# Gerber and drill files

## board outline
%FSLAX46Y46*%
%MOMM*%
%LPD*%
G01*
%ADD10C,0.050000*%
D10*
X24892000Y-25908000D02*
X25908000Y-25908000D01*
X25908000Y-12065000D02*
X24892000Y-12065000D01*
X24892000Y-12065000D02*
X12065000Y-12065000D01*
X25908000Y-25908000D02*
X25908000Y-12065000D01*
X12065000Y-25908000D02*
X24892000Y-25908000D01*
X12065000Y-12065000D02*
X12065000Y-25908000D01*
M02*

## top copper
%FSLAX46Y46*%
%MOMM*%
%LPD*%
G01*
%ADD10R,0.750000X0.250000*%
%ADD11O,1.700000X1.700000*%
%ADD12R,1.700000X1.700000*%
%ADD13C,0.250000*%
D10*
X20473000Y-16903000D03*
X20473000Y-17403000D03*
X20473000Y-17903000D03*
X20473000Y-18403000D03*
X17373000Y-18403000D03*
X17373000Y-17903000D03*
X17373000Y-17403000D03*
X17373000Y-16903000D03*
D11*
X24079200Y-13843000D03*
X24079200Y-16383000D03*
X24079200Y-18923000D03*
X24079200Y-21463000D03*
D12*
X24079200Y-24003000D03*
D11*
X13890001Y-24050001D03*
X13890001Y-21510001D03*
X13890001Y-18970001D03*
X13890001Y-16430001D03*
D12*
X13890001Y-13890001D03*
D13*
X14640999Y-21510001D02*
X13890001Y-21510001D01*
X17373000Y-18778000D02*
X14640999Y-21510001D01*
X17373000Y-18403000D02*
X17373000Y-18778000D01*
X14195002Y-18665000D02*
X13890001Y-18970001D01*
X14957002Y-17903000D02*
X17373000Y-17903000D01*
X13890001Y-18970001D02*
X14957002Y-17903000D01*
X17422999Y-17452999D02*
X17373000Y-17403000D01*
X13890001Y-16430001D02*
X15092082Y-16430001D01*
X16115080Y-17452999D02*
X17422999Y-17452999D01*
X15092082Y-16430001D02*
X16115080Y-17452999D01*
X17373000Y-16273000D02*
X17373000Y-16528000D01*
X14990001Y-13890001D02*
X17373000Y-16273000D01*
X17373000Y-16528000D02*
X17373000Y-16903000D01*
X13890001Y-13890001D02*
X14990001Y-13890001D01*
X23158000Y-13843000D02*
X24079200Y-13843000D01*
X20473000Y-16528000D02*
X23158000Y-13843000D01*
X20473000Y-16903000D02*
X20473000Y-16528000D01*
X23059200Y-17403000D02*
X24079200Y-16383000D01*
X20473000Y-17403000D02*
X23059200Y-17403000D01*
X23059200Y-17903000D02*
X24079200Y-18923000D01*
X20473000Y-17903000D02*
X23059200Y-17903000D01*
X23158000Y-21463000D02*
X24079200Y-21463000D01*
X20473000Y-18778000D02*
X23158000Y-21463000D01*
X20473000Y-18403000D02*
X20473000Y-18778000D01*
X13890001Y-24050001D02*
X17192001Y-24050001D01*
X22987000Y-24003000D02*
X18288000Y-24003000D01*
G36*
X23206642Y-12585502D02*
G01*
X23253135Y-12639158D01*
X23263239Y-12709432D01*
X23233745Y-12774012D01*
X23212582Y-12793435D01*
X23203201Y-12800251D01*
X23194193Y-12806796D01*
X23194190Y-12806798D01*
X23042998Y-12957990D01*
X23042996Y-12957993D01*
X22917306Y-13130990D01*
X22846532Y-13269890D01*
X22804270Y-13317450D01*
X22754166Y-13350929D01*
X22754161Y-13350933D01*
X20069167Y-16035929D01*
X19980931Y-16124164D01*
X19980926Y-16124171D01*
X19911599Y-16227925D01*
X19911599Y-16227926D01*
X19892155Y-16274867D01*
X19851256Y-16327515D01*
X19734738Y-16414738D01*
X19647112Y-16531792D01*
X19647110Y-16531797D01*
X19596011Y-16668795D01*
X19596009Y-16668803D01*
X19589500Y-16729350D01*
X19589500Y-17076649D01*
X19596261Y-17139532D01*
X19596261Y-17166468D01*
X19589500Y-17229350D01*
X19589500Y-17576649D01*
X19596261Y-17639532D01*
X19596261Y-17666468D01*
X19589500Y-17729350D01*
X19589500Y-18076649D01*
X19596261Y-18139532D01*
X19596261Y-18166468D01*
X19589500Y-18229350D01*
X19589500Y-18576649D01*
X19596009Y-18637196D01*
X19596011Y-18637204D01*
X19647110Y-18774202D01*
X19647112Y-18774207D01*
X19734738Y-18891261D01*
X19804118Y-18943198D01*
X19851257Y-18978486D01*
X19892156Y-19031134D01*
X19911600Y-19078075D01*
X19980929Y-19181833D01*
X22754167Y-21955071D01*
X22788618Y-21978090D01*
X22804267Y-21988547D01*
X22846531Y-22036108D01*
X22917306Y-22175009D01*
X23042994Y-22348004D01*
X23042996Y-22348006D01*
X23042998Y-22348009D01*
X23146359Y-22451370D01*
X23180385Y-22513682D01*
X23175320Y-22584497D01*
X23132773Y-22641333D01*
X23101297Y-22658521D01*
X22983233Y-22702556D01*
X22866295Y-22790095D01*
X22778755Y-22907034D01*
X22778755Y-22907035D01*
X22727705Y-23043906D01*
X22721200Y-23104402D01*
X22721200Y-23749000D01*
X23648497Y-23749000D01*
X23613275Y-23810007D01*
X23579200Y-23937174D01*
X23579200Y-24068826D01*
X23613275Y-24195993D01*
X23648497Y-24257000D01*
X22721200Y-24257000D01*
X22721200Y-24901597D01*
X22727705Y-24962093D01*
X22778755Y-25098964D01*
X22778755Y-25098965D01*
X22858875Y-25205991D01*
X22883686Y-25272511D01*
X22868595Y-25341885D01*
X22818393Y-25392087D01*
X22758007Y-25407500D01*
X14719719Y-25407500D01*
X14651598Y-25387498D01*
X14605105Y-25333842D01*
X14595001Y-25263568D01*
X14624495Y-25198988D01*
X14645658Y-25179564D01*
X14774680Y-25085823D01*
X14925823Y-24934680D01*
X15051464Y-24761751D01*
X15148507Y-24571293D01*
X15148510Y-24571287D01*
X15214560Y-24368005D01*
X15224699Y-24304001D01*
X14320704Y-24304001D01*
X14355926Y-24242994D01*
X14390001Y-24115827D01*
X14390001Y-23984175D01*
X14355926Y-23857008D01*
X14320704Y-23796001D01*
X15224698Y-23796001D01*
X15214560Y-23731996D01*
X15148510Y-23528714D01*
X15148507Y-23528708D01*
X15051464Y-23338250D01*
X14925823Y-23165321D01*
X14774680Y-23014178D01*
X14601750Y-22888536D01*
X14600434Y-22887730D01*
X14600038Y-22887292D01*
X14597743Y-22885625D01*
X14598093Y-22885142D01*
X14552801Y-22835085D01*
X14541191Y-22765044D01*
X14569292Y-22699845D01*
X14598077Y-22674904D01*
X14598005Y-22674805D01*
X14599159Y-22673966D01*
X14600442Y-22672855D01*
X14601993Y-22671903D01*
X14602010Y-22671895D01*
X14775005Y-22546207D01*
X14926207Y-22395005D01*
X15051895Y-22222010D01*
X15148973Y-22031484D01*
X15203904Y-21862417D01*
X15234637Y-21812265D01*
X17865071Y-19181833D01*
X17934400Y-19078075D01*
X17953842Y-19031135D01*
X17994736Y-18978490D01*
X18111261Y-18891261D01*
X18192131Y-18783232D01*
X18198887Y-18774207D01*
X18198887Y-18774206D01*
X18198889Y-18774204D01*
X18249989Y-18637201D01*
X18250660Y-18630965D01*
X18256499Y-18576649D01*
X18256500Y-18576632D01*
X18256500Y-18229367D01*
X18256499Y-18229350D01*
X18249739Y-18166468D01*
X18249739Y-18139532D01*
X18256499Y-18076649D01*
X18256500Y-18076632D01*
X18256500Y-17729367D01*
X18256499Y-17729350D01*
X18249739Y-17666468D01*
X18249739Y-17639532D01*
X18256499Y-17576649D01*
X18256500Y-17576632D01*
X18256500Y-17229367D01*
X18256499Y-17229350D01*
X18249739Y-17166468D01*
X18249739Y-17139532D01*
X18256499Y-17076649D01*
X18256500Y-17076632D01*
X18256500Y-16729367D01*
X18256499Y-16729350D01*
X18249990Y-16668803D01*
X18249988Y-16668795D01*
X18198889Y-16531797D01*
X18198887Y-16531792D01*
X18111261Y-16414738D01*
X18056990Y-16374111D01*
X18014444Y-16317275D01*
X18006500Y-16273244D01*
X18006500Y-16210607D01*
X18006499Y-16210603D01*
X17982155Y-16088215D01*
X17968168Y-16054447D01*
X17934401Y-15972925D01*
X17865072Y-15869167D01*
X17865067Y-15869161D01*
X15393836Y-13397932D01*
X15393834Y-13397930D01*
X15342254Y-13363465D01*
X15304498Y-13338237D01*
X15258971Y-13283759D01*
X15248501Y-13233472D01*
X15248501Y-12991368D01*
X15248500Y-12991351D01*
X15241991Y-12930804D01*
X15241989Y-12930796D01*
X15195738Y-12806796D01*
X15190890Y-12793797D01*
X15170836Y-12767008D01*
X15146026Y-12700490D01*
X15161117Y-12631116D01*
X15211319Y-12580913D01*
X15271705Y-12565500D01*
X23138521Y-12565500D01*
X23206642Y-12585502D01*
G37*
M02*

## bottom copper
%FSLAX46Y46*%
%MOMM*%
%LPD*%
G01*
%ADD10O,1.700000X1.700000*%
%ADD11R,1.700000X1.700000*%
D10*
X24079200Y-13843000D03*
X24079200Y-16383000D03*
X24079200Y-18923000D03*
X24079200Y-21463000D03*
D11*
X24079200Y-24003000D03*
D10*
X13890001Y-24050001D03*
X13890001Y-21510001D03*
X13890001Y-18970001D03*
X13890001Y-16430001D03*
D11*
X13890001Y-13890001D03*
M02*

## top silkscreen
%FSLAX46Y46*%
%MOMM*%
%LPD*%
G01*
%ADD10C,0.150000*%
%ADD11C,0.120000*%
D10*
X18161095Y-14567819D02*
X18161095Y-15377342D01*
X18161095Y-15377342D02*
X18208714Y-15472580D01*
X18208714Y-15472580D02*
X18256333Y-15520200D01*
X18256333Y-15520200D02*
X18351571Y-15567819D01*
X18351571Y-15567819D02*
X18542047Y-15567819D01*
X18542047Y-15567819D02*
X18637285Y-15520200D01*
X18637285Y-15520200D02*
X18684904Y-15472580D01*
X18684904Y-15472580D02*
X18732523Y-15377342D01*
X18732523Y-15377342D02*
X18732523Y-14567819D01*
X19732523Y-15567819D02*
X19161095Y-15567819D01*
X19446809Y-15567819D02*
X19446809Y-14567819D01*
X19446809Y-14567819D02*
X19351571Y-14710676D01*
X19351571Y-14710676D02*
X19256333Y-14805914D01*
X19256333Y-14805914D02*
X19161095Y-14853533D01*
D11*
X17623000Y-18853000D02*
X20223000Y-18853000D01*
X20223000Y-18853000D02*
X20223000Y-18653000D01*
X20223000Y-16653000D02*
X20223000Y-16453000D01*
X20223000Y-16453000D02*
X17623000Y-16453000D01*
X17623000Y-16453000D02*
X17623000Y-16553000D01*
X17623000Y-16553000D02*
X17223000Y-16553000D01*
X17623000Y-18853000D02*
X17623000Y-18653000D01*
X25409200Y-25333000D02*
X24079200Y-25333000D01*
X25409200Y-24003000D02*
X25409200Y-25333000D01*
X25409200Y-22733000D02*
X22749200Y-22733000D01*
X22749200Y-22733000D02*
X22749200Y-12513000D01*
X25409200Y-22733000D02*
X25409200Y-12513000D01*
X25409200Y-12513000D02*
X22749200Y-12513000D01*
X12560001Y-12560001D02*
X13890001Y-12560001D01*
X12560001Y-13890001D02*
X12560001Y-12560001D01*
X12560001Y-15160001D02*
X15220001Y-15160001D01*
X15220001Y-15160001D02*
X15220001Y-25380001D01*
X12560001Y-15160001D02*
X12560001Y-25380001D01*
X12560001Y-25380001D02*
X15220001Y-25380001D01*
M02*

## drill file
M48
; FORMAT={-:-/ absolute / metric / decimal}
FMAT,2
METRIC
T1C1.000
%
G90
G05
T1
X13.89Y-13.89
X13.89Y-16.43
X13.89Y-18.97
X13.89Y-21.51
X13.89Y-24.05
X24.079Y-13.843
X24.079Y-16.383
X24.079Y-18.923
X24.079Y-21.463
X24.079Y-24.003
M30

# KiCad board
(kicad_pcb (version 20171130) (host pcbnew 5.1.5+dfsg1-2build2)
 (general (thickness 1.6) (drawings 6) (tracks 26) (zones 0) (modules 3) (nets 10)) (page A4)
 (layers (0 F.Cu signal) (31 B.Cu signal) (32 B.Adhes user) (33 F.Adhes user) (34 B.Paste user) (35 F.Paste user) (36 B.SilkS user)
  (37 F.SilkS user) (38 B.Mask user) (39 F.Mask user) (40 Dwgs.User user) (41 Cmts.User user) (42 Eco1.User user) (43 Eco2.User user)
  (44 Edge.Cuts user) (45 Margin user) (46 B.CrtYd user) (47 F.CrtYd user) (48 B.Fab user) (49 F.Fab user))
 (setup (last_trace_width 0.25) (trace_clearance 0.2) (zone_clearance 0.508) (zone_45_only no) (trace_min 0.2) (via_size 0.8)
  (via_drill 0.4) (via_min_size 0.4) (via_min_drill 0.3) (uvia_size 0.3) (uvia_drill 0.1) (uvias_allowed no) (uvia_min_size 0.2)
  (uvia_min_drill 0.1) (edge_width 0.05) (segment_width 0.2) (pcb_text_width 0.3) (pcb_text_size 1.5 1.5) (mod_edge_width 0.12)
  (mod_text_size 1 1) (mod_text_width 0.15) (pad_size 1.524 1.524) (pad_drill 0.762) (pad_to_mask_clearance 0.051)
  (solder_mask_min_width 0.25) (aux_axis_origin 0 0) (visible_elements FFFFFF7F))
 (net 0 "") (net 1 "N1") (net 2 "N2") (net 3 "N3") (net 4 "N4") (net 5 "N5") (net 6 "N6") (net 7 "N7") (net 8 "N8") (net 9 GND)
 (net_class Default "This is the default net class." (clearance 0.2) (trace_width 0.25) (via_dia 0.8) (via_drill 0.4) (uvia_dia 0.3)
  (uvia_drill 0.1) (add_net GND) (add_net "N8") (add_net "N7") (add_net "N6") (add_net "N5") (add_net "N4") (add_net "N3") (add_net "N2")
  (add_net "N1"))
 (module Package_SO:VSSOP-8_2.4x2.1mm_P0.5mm (layer F.Cu) (at 18.923 17.653)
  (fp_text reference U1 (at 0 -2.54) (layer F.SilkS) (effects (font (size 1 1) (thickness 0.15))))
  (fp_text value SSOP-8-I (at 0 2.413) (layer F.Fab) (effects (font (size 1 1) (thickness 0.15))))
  (fp_line (start -1.3 1.2) (end 1.3 1.2) (layer F.SilkS) (width 0.12))
  (fp_line (start 1.3 1.2) (end 1.3 1) (layer F.SilkS) (width 0.12))
  (fp_line (start 1.3 -1) (end 1.3 -1.2) (layer F.SilkS) (width 0.12))
  (fp_line (start 1.3 -1.2) (end -1.3 -1.2) (layer F.SilkS) (width 0.12))
  (fp_line (start -1.3 -1.2) (end -1.3 -1.1) (layer F.SilkS) (width 0.12))
  (fp_line (start -1.3 -1.1) (end -1.7 -1.1) (layer F.SilkS) (width 0.12))
  (fp_line (start -1.3 1.2) (end -1.3 1) (layer F.SilkS) (width 0.12))
  (pad 8 smd rect (at 1.55 -0.75) (size 0.75 0.25) (layers F.Cu F.Paste F.Mask) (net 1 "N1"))
  (pad 7 smd rect (at 1.55 -0.25) (size 0.75 0.25) (layers F.Cu F.Paste F.Mask) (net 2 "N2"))
  (pad 6 smd rect (at 1.55 0.25) (size 0.75 0.25) (layers F.Cu F.Paste F.Mask) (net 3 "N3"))
  (pad 5 smd rect (at 1.55 0.75) (size 0.75 0.25) (layers F.Cu F.Paste F.Mask) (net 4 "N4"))
  (pad 4 smd rect (at -1.55 0.75) (size 0.75 0.25) (layers F.Cu F.Paste F.Mask) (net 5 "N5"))
  (pad 3 smd rect (at -1.55 0.25) (size 0.75 0.25) (layers F.Cu F.Paste F.Mask) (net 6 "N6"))
  (pad 2 smd rect (at -1.55 -0.25) (size 0.75 0.25) (layers F.Cu F.Paste F.Mask) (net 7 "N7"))
  (pad 1 smd rect (at -1.55 -0.75) (size 0.75 0.25) (layers F.Cu F.Paste F.Mask) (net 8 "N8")))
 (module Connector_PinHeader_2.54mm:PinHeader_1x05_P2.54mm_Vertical (layer F.Cu) (at 24.0792 24.003 180)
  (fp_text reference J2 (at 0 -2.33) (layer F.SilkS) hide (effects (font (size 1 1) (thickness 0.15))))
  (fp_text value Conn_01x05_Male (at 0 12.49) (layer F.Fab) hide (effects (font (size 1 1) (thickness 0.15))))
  (fp_line (start -1.33 -1.33) (end 0 -1.33) (layer F.SilkS) (width 0.12))
  (fp_line (start -1.33 0) (end -1.33 -1.33) (layer F.SilkS) (width 0.12))
  (fp_line (start -1.33 1.27) (end 1.33 1.27) (layer F.SilkS) (width 0.12))
  (fp_line (start 1.33 1.27) (end 1.33 11.49) (layer F.SilkS) (width 0.12))
  (fp_line (start -1.33 1.27) (end -1.33 11.49) (layer F.SilkS) (width 0.12))
  (fp_line (start -1.33 11.49) (end 1.33 11.49) (layer F.SilkS) (width 0.12))
  (pad 5 thru_hole oval (at 0 10.16 180) (size 1.7 1.7) (drill 1) (layers *.Cu *.Mask) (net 1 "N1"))
  (pad 4 thru_hole oval (at 0 7.62 180) (size 1.7 1.7) (drill 1) (layers *.Cu *.Mask) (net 2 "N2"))
  (pad 3 thru_hole oval (at 0 5.08 180) (size 1.7 1.7) (drill 1) (layers *.Cu *.Mask) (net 3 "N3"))
  (pad 2 thru_hole oval (at 0 2.54 180) (size 1.7 1.7) (drill 1) (layers *.Cu *.Mask) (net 4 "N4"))
  (pad 1 thru_hole rect (at 0 0 180) (size 1.7 1.7) (drill 1) (layers *.Cu *.Mask) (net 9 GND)))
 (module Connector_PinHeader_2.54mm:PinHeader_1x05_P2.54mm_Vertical (layer F.Cu) (at 13.890001 13.890001)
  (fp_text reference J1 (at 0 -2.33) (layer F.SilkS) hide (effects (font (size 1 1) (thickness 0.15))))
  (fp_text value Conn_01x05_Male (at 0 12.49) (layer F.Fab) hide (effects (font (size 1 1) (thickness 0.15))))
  (fp_line (start -1.33 -1.33) (end 0 -1.33) (layer F.SilkS) (width 0.12))
  (fp_line (start -1.33 0) (end -1.33 -1.33) (layer F.SilkS) (width 0.12))
  (fp_line (start -1.33 1.27) (end 1.33 1.27) (layer F.SilkS) (width 0.12))
  (fp_line (start 1.33 1.27) (end 1.33 11.49) (layer F.SilkS) (width 0.12))
  (fp_line (start -1.33 1.27) (end -1.33 11.49) (layer F.SilkS) (width 0.12))
  (fp_line (start -1.33 11.49) (end 1.33 11.49) (layer F.SilkS) (width 0.12))
  (pad 5 thru_hole oval (at 0 10.16) (size 1.7 1.7) (drill 1) (layers *.Cu *.Mask) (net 9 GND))
  (pad 4 thru_hole oval (at 0 7.62) (size 1.7 1.7) (drill 1) (layers *.Cu *.Mask) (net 5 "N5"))
  (pad 3 thru_hole oval (at 0 5.08) (size 1.7 1.7) (drill 1) (layers *.Cu *.Mask) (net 6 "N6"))
  (pad 2 thru_hole oval (at 0 2.54) (size 1.7 1.7) (drill 1) (layers *.Cu *.Mask) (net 7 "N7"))
  (pad 1 thru_hole rect (at 0 0) (size 1.7 1.7) (drill 1) (layers *.Cu *.Mask) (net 8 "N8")))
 (gr_line (start 24.892 25.908) (end 25.908 25.908) (layer Edge.Cuts) (width 0.05))
 (gr_line (start 25.908 12.065) (end 24.892 12.065) (layer Edge.Cuts) (width 0.05))
 (gr_line (start 24.892 12.065) (end 12.065 12.065) (layer Edge.Cuts) (width 0.05))
 (gr_line (start 25.908 25.908) (end 25.908 12.065) (layer Edge.Cuts) (width 0.05))
 (gr_line (start 12.065 25.908) (end 24.892 25.908) (layer Edge.Cuts) (width 0.05))
 (gr_line (start 12.065 12.065) (end 12.065 25.908) (layer Edge.Cuts) (width 0.05))
 (segment (start 14.640999 21.510001) (end 13.890001 21.510001) (width 0.25) (layer F.Cu) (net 5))
 (segment (start 17.373 18.778) (end 14.640999 21.510001) (width 0.25) (layer F.Cu) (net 5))
 (segment (start 17.373 18.403) (end 17.373 18.778) (width 0.25) (layer F.Cu) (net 5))
 (segment (start 14.195002 18.665) (end 13.890001 18.970001) (width 0.25) (layer F.Cu) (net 6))
 (segment (start 14.957002 17.903) (end 17.373 17.903) (width 0.25) (layer F.Cu) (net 6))
 (segment (start 13.890001 18.970001) (end 14.957002 17.903) (width 0.25) (layer F.Cu) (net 6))
 (segment (start 17.422999 17.452999) (end 17.373 17.403) (width 0.25) (layer F.Cu) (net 7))
 (segment (start 13.890001 16.430001) (end 15.092082 16.430001) (width 0.25) (layer F.Cu) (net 7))
 (segment (start 16.11508 17.452999) (end 17.422999 17.452999) (width 0.25) (layer F.Cu) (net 7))
 (segment (start 15.092082 16.430001) (end 16.11508 17.452999) (width 0.25) (layer F.Cu) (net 7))
 (segment (start 17.373 16.273) (end 17.373 16.528) (width 0.25) (layer F.Cu) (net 8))
 (segment (start 14.990001 13.890001) (end 17.373 16.273) (width 0.25) (layer F.Cu) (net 8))
 (segment (start 17.373 16.528) (end 17.373 16.903) (width 0.25) (layer F.Cu) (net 8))
 (segment (start 13.890001 13.890001) (end 14.990001 13.890001) (width 0.25) (layer F.Cu) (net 8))
 (segment (start 23.158 13.843) (end 24.0792 13.843) (width 0.25) (layer F.Cu) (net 1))
 (segment (start 20.473 16.528) (end 23.158 13.843) (width 0.25) (layer F.Cu) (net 1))
 (segment (start 20.473 16.903) (end 20.473 16.528) (width 0.25) (layer F.Cu) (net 1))
 (segment (start 23.0592 17.403) (end 24.0792 16.383) (width 0.25) (layer F.Cu) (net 2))
 (segment (start 20.473 17.403) (end 23.0592 17.403) (width 0.25) (layer F.Cu) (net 2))
 (segment (start 23.0592 17.903) (end 24.0792 18.923) (width 0.25) (layer F.Cu) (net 3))
 (segment (start 20.473 17.903) (end 23.0592 17.903) (width 0.25) (layer F.Cu) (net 3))
 (segment (start 23.158 21.463) (end 24.0792 21.463) (width 0.25) (layer F.Cu) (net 4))
 (segment (start 20.473 18.778) (end 23.158 21.463) (width 0.25) (layer F.Cu) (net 4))
 (segment (start 20.473 18.403) (end 20.473 18.778) (width 0.25) (layer F.Cu) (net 4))
 (segment (start 13.890001 24.050001) (end 17.192001 24.050001) (width 0.25) (layer F.Cu) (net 9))
 (segment (start 22.987 24.003) (end 18.288 24.003) (width 0.25) (layer F.Cu) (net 9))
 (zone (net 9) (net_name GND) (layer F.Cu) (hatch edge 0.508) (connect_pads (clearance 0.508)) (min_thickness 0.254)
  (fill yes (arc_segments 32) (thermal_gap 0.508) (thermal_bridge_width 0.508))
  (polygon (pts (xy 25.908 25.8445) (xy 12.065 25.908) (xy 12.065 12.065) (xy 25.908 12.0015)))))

